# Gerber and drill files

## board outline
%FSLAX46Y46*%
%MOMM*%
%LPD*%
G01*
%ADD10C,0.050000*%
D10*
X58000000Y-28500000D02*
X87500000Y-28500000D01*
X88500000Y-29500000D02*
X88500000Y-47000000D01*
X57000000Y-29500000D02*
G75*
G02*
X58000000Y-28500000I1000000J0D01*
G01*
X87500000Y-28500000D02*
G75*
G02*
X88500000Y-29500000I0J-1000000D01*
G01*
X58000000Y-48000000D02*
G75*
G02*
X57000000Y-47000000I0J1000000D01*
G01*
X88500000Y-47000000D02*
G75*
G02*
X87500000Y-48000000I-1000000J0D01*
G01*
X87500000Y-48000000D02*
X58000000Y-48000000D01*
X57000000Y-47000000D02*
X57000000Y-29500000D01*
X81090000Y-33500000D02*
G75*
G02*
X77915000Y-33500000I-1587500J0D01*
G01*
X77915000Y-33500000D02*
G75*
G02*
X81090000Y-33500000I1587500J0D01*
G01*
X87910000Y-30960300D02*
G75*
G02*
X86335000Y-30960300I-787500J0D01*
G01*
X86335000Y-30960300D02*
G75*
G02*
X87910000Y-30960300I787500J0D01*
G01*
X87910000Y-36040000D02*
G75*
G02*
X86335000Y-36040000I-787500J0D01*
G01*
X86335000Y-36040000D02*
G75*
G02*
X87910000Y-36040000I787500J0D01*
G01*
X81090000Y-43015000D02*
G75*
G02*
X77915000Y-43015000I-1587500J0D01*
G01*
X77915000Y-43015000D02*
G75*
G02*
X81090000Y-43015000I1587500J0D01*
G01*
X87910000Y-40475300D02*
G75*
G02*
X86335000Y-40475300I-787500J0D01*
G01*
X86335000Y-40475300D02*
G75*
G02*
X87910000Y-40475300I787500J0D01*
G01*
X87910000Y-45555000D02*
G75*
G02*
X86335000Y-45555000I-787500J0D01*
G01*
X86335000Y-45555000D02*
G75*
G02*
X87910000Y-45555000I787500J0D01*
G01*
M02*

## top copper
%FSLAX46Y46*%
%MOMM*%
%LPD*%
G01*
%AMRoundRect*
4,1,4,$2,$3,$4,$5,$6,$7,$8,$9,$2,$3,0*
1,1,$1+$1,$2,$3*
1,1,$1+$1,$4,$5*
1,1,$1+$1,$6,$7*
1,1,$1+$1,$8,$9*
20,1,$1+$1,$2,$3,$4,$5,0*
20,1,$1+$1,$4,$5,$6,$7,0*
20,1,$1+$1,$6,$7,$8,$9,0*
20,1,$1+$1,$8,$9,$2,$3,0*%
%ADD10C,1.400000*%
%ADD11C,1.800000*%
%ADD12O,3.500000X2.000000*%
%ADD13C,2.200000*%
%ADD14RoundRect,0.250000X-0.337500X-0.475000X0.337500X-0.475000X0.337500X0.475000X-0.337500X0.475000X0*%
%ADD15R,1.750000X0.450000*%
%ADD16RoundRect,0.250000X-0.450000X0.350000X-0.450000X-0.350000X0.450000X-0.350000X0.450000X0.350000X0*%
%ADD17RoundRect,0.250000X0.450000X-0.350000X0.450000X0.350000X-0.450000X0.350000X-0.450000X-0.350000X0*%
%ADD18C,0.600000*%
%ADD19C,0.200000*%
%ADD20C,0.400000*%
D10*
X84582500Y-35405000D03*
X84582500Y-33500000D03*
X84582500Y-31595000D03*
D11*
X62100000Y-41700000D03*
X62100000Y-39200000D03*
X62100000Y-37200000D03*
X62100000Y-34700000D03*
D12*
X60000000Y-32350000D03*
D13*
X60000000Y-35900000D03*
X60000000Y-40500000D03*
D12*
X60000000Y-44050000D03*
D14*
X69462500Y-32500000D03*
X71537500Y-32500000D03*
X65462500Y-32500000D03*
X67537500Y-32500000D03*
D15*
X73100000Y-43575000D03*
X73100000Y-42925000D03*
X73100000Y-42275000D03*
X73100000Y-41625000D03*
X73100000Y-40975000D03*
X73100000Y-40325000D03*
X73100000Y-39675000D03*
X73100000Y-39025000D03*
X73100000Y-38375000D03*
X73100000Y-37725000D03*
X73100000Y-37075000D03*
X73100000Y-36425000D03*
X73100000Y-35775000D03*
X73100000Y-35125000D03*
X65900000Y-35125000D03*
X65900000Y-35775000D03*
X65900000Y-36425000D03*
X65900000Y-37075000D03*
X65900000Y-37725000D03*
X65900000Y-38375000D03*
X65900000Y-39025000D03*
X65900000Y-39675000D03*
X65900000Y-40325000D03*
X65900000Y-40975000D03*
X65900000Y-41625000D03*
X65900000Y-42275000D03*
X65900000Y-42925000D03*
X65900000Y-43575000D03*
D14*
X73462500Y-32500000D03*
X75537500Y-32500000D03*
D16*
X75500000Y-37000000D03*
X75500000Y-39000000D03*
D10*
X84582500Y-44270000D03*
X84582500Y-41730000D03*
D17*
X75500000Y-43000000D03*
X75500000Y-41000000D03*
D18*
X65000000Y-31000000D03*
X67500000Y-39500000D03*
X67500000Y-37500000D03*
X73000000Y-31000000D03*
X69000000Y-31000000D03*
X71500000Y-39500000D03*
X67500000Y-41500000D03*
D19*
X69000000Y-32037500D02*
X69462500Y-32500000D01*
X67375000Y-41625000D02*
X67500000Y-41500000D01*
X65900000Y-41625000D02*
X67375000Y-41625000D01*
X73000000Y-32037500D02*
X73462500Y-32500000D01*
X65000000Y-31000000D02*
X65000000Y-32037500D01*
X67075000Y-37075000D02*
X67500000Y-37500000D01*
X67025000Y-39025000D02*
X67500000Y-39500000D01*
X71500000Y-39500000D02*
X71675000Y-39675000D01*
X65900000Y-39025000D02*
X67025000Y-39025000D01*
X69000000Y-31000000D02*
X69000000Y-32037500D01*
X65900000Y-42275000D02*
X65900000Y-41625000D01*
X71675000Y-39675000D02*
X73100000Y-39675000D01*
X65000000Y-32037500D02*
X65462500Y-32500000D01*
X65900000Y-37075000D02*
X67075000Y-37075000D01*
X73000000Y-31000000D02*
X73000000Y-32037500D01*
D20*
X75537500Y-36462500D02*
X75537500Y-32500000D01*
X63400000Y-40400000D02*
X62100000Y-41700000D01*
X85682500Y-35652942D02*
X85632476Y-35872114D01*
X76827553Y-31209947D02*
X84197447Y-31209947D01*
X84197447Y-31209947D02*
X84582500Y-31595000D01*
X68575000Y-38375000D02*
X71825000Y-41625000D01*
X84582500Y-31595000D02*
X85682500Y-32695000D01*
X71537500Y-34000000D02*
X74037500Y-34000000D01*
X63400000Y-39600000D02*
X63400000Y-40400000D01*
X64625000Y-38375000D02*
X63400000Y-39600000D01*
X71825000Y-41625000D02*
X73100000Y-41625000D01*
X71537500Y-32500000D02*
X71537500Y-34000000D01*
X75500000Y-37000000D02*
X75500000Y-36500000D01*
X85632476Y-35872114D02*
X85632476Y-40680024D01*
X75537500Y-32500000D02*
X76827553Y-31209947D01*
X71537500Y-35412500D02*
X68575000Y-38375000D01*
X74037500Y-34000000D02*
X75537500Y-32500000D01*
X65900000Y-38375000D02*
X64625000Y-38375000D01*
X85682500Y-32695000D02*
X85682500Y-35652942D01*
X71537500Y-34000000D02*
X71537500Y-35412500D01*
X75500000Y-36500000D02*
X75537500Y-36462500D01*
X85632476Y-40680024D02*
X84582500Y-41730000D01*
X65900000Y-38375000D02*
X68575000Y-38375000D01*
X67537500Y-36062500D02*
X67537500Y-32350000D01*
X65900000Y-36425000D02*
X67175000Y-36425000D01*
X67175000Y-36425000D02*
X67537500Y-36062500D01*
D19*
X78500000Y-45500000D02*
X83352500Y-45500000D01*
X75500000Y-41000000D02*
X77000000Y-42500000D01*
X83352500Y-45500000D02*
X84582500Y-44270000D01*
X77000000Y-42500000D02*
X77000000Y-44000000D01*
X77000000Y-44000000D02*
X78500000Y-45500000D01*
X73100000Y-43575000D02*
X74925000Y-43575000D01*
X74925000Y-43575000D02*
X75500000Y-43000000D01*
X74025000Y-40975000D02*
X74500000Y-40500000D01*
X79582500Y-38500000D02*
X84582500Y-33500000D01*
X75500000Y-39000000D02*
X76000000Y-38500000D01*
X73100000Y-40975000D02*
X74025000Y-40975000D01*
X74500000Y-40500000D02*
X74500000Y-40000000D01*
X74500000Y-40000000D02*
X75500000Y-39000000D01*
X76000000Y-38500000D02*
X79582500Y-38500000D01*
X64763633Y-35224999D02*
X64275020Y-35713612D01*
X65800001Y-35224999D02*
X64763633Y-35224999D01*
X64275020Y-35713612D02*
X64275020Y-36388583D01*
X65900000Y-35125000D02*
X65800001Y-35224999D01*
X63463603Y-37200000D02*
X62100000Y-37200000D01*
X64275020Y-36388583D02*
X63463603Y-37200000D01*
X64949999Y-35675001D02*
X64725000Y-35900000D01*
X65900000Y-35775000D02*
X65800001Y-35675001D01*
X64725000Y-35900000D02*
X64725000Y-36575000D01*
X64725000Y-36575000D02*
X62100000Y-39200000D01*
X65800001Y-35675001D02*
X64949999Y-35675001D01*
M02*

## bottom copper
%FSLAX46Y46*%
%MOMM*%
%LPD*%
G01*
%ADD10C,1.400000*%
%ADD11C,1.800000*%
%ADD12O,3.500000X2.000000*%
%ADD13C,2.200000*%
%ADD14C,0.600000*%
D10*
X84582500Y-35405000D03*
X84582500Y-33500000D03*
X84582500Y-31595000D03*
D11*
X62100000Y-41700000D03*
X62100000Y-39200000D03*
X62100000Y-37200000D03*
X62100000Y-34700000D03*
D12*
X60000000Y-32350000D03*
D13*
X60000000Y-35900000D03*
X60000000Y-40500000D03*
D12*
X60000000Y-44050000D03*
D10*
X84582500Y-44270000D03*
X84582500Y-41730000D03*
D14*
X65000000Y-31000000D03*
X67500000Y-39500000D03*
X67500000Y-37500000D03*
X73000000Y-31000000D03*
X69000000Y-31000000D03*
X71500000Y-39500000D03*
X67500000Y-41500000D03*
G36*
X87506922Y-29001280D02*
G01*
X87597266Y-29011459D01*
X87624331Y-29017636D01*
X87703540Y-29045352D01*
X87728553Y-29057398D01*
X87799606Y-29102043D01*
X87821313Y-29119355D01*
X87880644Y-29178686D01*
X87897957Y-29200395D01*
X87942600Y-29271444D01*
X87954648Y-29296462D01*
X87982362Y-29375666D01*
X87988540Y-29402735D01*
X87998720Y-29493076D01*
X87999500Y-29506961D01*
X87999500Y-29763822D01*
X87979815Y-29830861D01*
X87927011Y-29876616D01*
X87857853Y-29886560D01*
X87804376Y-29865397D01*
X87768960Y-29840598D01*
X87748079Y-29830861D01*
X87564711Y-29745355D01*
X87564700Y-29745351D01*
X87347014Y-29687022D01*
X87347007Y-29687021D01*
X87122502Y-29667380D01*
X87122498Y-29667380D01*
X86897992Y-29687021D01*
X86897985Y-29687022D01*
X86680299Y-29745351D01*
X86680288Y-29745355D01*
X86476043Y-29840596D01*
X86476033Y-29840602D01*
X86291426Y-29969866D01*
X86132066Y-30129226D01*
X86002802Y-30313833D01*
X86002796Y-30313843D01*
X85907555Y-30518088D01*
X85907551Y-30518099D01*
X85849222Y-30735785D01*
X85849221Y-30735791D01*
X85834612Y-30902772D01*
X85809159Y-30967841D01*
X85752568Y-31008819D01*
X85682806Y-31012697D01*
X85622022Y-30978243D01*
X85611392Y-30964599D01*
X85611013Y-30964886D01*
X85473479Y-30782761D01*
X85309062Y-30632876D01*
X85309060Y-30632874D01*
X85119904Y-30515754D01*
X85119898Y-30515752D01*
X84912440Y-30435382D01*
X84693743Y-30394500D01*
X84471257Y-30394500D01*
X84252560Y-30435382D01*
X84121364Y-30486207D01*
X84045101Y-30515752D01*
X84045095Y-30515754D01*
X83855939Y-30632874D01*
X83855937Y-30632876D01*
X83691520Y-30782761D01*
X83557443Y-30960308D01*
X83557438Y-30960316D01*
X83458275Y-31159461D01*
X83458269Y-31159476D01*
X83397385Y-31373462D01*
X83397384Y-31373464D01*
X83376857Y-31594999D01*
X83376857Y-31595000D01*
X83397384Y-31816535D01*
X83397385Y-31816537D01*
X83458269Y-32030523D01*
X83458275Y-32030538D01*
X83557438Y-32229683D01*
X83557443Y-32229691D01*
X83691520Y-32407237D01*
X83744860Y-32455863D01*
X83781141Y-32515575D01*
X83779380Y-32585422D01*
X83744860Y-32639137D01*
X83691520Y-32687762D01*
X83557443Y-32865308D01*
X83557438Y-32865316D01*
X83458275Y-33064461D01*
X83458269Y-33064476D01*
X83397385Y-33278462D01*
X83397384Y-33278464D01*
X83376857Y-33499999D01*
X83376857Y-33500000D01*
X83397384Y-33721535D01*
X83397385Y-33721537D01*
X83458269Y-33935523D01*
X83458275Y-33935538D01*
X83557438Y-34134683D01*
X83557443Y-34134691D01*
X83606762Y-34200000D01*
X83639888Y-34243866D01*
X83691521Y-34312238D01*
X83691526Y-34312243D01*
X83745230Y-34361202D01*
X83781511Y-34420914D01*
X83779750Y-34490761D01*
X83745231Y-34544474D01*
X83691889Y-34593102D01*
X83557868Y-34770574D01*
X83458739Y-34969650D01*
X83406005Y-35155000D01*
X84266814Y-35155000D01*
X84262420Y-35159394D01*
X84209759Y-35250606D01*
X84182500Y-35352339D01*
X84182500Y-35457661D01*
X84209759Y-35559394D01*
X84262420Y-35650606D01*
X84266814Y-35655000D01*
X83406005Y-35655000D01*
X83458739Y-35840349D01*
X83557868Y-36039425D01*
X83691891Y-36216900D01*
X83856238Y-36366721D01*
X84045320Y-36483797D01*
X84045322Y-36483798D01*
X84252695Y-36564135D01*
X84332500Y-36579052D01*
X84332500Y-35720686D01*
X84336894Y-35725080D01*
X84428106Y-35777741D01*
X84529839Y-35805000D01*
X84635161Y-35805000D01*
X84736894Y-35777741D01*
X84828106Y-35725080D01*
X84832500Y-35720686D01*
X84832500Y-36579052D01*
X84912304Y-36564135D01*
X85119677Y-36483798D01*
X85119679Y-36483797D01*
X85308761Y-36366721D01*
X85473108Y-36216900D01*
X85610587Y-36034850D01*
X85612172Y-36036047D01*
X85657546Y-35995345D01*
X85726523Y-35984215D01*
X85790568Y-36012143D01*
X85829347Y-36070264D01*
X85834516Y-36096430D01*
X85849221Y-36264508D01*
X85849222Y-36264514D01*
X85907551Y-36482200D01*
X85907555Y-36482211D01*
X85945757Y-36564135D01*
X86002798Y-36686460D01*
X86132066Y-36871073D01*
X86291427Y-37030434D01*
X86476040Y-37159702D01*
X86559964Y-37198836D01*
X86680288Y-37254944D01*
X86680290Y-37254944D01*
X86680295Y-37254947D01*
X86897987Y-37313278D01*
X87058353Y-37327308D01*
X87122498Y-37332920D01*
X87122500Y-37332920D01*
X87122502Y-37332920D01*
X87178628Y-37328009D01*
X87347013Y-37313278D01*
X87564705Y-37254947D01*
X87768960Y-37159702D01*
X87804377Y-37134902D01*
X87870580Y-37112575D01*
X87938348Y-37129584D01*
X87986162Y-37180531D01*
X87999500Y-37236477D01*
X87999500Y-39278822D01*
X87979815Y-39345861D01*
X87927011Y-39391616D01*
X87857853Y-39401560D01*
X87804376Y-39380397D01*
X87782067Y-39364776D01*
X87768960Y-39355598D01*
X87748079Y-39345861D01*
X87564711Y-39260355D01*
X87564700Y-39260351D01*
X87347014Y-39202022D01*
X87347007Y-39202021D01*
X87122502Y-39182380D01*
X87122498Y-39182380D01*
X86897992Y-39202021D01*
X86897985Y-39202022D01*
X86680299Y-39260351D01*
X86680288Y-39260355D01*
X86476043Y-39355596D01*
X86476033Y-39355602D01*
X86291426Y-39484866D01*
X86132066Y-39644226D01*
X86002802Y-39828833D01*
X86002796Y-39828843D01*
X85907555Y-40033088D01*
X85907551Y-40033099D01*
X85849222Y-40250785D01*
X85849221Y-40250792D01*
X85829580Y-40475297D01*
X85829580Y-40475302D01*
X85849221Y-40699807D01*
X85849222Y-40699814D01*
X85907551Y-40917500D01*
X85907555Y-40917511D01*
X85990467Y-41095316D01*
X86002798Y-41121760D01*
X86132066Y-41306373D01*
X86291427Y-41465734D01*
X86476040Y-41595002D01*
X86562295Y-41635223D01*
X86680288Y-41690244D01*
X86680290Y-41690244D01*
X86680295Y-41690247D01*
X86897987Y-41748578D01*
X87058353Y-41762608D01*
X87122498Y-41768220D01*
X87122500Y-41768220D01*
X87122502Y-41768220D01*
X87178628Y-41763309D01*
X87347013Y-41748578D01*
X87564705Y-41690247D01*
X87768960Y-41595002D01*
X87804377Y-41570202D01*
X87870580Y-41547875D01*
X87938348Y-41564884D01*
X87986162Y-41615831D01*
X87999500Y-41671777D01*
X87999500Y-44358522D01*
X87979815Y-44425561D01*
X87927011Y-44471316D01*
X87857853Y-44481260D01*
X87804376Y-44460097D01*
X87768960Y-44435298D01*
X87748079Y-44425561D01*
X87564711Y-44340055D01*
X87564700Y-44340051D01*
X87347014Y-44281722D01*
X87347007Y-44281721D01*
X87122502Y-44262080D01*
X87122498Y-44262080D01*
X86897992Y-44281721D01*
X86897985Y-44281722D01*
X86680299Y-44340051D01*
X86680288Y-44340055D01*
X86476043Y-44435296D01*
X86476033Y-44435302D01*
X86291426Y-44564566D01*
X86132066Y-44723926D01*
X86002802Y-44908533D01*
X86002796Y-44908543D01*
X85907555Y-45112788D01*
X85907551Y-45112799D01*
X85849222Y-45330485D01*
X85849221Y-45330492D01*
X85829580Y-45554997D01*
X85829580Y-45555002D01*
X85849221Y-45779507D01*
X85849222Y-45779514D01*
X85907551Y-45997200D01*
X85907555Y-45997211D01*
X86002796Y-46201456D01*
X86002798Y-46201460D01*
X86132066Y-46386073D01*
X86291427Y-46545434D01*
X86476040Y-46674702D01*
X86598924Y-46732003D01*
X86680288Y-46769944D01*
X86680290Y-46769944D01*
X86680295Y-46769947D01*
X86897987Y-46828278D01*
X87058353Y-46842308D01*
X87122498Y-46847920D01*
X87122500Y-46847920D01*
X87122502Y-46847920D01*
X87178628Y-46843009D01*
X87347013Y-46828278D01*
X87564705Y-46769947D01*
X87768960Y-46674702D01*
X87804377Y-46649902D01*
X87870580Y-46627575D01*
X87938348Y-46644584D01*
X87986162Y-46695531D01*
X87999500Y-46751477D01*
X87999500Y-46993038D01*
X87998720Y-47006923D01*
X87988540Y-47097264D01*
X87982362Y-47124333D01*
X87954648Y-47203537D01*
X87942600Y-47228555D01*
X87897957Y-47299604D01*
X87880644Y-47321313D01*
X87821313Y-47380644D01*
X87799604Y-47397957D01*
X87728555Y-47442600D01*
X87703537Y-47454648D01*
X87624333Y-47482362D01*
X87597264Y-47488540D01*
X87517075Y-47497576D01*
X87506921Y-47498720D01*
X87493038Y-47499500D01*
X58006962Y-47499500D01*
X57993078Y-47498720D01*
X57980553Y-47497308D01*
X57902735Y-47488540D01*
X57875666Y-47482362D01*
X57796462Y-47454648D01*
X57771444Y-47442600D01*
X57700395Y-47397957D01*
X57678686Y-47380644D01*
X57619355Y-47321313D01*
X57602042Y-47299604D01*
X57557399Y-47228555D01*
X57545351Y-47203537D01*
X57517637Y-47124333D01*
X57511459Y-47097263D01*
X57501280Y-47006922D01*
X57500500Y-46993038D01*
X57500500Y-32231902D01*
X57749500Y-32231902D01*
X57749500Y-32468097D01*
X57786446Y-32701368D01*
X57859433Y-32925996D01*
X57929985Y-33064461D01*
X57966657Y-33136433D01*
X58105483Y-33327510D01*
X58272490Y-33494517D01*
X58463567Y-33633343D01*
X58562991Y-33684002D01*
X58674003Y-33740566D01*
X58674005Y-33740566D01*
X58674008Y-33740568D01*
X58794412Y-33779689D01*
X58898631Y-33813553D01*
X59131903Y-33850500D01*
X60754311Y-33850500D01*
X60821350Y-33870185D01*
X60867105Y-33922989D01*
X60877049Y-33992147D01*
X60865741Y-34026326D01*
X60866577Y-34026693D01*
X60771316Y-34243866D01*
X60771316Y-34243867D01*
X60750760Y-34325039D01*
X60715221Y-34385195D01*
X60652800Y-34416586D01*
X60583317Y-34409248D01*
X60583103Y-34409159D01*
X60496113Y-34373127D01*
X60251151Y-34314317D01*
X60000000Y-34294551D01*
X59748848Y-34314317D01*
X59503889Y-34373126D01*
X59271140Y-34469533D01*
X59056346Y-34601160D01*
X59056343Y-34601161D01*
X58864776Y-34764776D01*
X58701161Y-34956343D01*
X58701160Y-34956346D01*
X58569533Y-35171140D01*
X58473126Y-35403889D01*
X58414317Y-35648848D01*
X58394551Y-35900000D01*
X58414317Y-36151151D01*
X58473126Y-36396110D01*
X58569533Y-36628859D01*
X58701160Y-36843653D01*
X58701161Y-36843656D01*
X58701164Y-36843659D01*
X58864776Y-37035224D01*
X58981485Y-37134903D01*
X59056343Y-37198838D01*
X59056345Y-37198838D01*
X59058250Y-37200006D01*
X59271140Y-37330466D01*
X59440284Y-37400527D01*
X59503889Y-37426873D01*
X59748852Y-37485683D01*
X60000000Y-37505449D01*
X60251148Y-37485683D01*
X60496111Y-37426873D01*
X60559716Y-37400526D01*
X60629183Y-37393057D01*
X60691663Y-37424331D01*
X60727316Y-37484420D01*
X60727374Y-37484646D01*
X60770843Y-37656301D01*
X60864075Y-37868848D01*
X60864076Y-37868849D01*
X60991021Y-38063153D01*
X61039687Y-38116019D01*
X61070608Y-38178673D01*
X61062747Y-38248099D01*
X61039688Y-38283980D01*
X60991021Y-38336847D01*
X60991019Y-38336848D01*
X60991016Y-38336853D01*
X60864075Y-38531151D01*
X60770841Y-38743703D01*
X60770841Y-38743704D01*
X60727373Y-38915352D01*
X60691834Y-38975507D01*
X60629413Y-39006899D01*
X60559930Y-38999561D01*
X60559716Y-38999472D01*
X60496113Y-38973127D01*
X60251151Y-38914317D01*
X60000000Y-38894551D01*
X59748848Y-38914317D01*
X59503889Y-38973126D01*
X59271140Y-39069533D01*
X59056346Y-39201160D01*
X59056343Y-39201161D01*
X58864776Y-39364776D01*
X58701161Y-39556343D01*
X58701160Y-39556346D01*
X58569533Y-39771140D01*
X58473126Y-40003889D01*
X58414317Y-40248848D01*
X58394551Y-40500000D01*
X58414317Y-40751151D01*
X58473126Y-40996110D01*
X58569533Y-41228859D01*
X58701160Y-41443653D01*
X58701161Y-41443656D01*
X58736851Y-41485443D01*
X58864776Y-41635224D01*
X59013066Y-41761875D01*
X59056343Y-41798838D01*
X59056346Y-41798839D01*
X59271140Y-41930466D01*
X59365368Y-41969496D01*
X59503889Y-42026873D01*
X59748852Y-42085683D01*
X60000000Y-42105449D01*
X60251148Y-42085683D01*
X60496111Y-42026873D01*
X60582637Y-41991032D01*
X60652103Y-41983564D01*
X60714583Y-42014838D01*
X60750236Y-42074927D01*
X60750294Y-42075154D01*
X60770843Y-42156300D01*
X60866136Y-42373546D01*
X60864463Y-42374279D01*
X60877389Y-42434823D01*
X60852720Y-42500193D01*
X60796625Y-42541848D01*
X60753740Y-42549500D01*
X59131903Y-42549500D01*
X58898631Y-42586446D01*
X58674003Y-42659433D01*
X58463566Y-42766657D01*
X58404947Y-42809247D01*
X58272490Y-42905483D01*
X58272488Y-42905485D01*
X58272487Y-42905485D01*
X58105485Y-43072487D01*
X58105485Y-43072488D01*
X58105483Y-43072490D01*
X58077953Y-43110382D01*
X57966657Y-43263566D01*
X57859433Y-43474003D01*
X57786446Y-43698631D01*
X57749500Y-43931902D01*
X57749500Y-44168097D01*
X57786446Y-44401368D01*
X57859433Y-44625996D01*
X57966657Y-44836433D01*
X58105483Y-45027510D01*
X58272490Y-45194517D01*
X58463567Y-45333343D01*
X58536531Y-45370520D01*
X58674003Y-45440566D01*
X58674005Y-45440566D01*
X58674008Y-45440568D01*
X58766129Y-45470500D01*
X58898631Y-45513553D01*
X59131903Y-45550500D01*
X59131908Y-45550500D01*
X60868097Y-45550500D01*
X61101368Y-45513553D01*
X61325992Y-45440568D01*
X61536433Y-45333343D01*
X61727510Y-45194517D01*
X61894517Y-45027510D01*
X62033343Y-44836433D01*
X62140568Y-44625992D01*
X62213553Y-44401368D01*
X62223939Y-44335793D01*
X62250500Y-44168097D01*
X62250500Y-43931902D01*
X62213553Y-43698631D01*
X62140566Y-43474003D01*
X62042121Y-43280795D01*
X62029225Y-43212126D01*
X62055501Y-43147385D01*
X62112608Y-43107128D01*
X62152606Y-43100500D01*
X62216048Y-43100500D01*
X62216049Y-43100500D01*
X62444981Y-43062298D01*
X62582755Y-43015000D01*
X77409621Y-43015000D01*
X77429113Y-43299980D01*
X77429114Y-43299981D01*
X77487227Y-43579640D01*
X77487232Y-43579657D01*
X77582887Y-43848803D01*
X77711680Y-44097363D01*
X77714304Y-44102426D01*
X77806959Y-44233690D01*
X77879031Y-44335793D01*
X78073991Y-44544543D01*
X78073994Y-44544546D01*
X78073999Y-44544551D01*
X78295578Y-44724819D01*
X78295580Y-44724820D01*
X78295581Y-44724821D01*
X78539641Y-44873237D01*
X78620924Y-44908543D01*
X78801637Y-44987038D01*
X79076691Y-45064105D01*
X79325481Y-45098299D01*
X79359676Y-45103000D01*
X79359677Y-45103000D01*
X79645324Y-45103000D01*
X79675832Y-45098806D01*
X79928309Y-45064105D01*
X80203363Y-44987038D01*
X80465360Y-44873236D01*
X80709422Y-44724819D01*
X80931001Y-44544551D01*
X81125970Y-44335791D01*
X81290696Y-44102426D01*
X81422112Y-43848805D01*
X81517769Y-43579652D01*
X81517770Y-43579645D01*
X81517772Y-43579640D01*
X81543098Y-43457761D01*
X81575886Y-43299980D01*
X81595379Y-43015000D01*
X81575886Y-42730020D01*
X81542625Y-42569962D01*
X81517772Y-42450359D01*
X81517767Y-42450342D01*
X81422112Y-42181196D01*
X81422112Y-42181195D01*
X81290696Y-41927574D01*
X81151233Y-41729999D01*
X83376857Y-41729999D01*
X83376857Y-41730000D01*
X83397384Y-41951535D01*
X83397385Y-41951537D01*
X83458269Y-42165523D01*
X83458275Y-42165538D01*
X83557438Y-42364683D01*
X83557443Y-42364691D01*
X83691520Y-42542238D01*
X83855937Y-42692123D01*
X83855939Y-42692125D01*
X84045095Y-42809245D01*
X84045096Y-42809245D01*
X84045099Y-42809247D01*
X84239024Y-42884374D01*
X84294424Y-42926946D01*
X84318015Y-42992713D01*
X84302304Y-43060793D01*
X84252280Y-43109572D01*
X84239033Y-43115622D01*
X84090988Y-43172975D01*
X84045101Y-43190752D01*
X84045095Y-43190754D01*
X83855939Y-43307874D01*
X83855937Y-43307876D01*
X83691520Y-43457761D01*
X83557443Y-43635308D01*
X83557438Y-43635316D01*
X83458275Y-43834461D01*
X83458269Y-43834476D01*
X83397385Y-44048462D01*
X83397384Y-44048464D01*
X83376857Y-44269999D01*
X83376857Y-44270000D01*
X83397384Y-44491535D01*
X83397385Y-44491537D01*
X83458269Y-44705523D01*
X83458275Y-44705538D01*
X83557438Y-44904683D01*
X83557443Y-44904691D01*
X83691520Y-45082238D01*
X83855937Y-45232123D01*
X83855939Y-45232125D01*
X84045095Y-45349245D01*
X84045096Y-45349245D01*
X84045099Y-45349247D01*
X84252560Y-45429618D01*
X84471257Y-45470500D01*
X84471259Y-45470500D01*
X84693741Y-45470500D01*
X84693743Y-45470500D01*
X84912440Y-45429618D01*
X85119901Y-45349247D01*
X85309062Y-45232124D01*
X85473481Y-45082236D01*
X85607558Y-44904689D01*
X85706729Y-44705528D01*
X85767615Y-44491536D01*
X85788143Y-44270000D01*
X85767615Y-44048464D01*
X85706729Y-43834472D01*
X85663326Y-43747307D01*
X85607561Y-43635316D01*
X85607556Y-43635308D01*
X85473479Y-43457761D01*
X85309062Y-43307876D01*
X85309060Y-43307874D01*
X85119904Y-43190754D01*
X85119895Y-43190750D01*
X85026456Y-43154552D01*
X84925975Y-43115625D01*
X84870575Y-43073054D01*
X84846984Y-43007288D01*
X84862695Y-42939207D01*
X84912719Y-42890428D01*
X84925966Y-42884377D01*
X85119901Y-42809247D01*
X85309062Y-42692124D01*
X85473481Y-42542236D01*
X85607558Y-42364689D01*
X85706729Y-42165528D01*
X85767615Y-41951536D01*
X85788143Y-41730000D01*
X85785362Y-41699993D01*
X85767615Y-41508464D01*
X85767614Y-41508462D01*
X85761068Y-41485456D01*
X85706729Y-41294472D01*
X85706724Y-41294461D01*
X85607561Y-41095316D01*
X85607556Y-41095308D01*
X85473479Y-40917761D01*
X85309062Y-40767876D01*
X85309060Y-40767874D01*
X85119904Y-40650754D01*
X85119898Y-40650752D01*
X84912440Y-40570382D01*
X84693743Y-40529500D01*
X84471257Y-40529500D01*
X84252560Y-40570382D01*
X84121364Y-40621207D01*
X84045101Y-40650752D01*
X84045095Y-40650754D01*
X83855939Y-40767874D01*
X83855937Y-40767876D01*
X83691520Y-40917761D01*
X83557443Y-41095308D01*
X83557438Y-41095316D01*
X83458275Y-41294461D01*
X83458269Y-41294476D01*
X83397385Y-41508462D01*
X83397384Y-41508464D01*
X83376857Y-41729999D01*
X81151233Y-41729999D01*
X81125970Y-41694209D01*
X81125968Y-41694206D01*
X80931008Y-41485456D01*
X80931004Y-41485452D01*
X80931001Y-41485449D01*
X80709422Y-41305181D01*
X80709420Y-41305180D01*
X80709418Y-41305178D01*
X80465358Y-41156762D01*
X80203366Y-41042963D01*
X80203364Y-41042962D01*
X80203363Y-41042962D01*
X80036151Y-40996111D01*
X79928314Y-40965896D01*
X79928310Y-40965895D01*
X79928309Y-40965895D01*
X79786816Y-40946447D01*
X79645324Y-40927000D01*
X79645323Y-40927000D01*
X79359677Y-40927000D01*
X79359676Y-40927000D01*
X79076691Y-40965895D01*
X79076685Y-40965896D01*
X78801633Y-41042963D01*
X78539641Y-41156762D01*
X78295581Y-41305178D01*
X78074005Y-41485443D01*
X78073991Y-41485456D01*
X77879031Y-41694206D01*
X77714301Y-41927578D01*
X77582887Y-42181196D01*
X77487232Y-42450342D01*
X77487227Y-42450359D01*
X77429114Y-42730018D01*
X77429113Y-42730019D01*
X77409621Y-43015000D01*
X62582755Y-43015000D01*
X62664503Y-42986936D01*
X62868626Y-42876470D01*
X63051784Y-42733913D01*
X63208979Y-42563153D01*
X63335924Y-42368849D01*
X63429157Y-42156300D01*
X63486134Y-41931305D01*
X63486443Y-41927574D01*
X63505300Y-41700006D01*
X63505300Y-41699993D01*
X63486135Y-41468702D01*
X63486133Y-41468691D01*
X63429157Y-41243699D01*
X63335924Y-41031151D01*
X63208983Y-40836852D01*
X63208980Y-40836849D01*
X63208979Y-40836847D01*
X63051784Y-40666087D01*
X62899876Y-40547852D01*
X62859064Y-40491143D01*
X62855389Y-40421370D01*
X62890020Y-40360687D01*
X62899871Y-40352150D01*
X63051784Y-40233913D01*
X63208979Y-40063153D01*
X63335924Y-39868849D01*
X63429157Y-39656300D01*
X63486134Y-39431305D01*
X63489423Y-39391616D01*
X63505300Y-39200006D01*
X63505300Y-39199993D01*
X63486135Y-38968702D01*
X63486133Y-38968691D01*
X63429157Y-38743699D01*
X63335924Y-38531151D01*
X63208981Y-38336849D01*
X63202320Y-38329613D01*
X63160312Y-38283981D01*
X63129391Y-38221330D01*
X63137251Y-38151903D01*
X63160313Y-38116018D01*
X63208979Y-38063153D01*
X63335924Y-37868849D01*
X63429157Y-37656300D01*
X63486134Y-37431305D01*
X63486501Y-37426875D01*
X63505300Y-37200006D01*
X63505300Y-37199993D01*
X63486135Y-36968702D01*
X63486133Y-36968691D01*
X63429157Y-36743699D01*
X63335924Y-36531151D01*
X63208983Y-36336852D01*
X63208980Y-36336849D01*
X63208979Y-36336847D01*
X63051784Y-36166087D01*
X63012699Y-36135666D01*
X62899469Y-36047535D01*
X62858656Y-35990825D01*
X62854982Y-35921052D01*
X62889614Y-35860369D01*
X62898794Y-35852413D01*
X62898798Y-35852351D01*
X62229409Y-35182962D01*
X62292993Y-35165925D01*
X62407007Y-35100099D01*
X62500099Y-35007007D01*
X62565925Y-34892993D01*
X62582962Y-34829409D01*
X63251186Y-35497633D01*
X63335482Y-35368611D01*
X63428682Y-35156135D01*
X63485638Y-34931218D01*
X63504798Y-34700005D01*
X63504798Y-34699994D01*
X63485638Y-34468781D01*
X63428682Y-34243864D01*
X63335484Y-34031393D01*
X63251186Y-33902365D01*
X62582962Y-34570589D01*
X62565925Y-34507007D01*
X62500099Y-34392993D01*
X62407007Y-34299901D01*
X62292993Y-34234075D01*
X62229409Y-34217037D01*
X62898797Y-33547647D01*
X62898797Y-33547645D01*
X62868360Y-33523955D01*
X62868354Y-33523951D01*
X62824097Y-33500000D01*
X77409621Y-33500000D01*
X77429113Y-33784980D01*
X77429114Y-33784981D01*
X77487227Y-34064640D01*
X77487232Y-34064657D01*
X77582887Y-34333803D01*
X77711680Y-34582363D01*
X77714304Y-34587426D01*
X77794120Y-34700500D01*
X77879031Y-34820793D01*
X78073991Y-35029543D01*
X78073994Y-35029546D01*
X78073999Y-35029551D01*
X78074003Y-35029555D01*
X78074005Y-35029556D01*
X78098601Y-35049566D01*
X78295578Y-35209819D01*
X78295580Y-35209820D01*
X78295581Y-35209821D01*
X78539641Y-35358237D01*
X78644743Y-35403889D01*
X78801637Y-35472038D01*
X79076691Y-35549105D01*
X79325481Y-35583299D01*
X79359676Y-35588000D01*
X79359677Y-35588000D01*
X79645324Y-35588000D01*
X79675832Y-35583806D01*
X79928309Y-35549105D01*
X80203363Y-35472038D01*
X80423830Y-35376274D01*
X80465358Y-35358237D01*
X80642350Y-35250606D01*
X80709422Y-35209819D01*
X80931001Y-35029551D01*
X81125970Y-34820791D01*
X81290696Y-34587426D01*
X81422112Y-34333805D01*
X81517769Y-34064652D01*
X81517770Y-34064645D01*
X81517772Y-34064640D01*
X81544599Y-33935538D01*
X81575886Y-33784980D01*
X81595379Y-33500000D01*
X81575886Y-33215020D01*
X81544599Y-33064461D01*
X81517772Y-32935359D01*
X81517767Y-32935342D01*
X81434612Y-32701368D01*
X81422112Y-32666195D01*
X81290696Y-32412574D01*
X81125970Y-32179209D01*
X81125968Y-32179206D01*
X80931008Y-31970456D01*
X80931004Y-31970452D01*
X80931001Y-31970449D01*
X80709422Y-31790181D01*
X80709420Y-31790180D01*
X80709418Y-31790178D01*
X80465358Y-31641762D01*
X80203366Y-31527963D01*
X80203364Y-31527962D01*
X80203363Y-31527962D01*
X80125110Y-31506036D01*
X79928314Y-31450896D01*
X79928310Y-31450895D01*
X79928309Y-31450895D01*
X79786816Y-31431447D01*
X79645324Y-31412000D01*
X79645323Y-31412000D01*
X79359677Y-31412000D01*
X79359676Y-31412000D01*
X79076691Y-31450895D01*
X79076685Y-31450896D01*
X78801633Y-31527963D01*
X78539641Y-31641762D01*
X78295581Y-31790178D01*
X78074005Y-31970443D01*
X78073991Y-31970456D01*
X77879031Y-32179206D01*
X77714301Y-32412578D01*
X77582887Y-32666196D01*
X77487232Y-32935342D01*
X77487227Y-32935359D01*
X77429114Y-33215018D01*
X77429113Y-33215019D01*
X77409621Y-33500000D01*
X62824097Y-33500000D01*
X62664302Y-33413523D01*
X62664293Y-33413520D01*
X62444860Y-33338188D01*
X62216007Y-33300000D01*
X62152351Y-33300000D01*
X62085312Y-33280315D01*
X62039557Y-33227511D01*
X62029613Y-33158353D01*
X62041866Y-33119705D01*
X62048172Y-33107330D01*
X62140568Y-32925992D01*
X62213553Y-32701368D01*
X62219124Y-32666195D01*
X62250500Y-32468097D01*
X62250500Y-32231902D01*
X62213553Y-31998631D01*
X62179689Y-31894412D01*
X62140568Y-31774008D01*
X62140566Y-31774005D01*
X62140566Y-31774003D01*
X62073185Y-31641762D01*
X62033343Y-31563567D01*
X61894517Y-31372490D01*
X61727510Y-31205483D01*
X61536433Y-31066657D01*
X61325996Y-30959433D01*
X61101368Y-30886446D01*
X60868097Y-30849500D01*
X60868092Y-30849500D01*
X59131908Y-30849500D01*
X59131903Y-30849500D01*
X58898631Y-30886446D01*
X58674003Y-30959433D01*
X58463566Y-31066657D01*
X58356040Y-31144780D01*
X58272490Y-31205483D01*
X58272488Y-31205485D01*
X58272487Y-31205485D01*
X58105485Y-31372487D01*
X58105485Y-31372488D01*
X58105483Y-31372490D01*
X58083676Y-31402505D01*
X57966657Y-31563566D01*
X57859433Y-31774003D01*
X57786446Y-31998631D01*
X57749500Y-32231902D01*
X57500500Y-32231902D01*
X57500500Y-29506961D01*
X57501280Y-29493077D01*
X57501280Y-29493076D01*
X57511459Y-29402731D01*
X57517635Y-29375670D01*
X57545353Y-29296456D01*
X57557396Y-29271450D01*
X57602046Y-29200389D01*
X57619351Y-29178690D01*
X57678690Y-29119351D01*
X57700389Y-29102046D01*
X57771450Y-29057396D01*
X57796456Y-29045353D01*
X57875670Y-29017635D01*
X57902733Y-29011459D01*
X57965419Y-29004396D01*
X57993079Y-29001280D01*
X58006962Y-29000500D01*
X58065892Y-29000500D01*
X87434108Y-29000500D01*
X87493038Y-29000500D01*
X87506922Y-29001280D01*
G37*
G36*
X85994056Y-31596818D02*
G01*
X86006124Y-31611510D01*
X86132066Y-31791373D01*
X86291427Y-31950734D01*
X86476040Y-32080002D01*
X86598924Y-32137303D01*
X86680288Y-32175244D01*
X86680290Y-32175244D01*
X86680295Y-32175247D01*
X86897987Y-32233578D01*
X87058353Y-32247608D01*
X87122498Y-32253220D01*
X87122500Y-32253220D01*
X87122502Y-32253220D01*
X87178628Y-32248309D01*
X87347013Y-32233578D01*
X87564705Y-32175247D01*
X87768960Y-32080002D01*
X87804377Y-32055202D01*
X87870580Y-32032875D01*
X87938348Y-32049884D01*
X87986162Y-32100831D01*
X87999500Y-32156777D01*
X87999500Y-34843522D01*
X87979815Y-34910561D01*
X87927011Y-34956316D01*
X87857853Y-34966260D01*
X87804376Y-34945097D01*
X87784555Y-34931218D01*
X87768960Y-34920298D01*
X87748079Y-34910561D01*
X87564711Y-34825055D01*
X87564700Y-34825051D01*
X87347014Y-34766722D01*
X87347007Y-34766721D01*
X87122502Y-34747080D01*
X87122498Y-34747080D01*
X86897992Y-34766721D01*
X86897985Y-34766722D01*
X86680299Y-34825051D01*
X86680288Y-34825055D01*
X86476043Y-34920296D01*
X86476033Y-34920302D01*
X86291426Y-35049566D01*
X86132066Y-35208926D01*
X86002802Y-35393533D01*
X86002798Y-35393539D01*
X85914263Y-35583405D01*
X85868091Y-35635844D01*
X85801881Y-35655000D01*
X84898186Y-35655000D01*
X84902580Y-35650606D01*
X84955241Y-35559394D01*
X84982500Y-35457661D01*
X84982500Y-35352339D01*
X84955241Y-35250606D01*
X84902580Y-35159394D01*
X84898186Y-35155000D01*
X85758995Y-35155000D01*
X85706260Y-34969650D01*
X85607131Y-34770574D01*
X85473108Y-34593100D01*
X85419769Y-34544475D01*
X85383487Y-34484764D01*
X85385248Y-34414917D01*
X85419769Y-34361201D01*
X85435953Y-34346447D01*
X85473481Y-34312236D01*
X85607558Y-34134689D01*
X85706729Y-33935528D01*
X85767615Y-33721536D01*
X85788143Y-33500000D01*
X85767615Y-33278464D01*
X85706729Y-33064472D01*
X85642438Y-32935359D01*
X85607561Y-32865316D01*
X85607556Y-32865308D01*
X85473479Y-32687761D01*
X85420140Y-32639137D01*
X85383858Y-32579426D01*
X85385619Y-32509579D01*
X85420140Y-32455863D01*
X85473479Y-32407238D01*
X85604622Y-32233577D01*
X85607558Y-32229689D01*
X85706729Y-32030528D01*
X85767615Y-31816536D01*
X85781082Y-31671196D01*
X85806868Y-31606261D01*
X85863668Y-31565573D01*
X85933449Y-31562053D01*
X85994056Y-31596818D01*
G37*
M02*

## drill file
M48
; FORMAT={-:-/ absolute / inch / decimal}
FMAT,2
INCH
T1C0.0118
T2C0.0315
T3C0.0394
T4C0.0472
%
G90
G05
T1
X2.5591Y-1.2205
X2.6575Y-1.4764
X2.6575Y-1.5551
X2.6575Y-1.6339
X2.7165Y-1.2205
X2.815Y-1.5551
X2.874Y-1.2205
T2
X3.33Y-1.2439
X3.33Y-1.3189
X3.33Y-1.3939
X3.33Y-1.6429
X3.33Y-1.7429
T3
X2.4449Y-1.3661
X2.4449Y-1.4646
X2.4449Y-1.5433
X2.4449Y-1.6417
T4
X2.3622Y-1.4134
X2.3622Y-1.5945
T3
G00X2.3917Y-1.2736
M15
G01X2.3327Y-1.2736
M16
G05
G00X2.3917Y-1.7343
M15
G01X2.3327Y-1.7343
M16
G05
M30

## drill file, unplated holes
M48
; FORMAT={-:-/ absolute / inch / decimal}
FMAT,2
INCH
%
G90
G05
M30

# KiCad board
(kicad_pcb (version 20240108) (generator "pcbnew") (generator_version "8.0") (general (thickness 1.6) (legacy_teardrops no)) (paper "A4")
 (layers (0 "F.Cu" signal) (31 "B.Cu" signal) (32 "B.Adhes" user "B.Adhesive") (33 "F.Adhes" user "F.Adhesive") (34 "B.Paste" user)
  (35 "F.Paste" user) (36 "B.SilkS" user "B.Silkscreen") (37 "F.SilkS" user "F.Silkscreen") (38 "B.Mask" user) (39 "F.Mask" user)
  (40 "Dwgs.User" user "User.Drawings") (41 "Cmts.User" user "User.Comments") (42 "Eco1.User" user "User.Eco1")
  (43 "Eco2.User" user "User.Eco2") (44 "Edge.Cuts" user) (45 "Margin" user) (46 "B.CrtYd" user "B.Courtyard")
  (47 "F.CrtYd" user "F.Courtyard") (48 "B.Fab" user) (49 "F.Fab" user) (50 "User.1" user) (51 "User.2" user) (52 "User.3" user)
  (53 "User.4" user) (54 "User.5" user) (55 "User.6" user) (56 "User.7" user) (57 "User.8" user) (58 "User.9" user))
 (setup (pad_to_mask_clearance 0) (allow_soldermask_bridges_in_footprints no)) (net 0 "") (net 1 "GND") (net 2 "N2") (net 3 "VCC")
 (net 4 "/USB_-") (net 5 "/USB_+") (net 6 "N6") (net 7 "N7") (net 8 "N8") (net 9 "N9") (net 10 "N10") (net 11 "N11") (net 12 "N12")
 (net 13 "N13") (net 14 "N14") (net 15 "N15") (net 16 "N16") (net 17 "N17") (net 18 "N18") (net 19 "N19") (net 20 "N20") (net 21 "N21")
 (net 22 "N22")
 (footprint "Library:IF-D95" (layer "F.Cu") (at 88.0675 30.0075 -90)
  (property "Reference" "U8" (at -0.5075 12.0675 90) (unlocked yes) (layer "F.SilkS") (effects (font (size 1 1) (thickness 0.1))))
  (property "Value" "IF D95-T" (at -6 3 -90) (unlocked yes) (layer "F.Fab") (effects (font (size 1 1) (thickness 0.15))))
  (fp_circle (center 3.4925 8.565) (end 5.08 8.565) (stroke (width 0.05) (type default)) (fill none) (layer "Edge.Cuts"))
  (fp_circle (center 0.9528 0.945) (end 1.7403 0.945) (stroke (width 0.05) (type default)) (fill none) (layer "Edge.Cuts"))
  (fp_circle (center 6.0325 0.945) (end 6.82 0.945) (stroke (width 0.05) (type default)) (fill none) (layer "Edge.Cuts"))
  (pad "1" thru_hole circle (at 5.3975 3.485 270) (size 1.4 1.4) (drill 0.8) (layers "*.Cu" "*.Mask") (remove_unused_layers no)
   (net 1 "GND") (thermal_bridge_angle 90))
  (pad "2" thru_hole circle (at 3.4925 3.485 270) (size 1.4 1.4) (drill 0.8) (layers "*.Cu" "*.Mask") (remove_unused_layers no) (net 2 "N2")
   (thermal_bridge_angle 90))
  (pad "3" thru_hole circle (at 1.5875 3.485 270) (size 1.4 1.4) (drill 0.8) (layers "*.Cu" "*.Mask") (remove_unused_layers no)
   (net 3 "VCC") (thermal_bridge_angle 90)))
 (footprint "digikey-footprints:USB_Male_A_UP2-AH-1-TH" (layer "F.Cu") (at 60 38.2 -90)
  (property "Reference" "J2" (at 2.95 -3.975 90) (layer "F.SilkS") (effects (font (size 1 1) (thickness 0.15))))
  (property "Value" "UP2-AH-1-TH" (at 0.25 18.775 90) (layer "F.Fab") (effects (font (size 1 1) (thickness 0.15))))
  (pad "1" thru_hole circle (at 3.5 -2.1 270) (size 1.8 1.8) (drill 1) (layers "*.Cu" "*.Mask") (remove_unused_layers no) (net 3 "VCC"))
  (pad "2" thru_hole circle (at 1 -2.1 270) (size 1.8 1.8) (drill 1) (layers "*.Cu" "*.Mask") (remove_unused_layers no) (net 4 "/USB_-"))
  (pad "3" thru_hole circle (at -1 -2.1 270) (size 1.8 1.8) (drill 1) (layers "*.Cu" "*.Mask") (remove_unused_layers no) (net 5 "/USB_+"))
  (pad "4" thru_hole circle (at -3.5 -2.1 270) (size 1.8 1.8) (drill 1) (layers "*.Cu" "*.Mask") (remove_unused_layers no) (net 1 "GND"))
  (pad "SH" thru_hole oval (at -5.85 0 270) (size 2 3.5) (drill oval 1 2.5) (layers "*.Cu" "*.Mask") (remove_unused_layers no))
  (pad "SH" thru_hole circle (at -2.3 0 270) (size 2.2 2.2) (drill 1.2) (layers "*.Cu" "*.Mask") (remove_unused_layers no))
  (pad "SH" thru_hole circle (at 2.3 0 270) (size 2.2 2.2) (drill 1.2) (layers "*.Cu" "*.Mask") (remove_unused_layers no))
  (pad "SH" thru_hole oval (at 5.85 0 270) (size 2 3.5) (drill oval 1 2.5) (layers "*.Cu" "*.Mask") (remove_unused_layers no)))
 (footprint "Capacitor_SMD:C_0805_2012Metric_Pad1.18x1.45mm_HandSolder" (layer "F.Cu") (at 70.5 32.5)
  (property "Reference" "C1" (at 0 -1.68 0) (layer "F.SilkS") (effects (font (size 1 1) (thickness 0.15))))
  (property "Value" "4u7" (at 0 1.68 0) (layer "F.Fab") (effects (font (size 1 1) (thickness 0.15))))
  (pad "1" smd roundrect (at -1.0375 0) (size 1.175 1.45) (layers "F.Cu" "F.Paste" "F.Mask") (roundrect_rratio 0.212766) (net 1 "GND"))
  (pad "2" smd roundrect (at 1.0375 0) (size 1.175 1.45) (layers "F.Cu" "F.Paste" "F.Mask") (roundrect_rratio 0.212766) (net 3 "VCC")))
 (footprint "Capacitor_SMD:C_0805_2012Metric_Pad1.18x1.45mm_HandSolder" (layer "F.Cu") (at 66.5 32.5)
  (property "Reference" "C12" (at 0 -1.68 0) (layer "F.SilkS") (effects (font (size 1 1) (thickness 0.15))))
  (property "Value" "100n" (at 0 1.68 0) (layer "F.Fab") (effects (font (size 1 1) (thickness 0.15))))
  (pad "1" smd roundrect (at -1.0375 0) (size 1.175 1.45) (layers "F.Cu" "F.Paste" "F.Mask") (roundrect_rratio 0.212766) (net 1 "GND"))
  (pad "2" smd roundrect (at 1.0375 0) (size 1.175 1.45) (layers "F.Cu" "F.Paste" "F.Mask") (roundrect_rratio 0.212766) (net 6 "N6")))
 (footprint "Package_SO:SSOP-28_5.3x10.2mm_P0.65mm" (layer "F.Cu") (at 69.5 39.35 180)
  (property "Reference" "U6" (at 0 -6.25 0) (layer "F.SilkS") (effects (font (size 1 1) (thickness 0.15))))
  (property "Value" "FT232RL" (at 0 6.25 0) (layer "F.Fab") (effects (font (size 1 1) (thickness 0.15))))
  (pad "1" smd rect (at -3.6 -4.225 180) (size 1.75 0.45) (layers "F.Cu" "F.Paste" "F.Mask") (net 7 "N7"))
  (pad "2" smd rect (at -3.6 -3.575 180) (size 1.75 0.45) (layers "F.Cu" "F.Paste" "F.Mask") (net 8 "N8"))
  (pad "3" smd rect (at -3.6 -2.925 180) (size 1.75 0.45) (layers "F.Cu" "F.Paste" "F.Mask") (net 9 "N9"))
  (pad "4" smd rect (at -3.6 -2.275 180) (size 1.75 0.45) (layers "F.Cu" "F.Paste" "F.Mask") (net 3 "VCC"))
  (pad "5" smd rect (at -3.6 -1.625 180) (size 1.75 0.45) (layers "F.Cu" "F.Paste" "F.Mask") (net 2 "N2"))
  (pad "6" smd rect (at -3.6 -0.975 180) (size 1.75 0.45) (layers "F.Cu" "F.Paste" "F.Mask") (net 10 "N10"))
  (pad "7" smd rect (at -3.6 -0.325 180) (size 1.75 0.45) (layers "F.Cu" "F.Paste" "F.Mask") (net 1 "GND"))
  (pad "8" smd rect (at -3.6 0.325 180) (size 1.75 0.45) (layers "F.Cu" "F.Paste" "F.Mask"))
  (pad "9" smd rect (at -3.6 0.975 180) (size 1.75 0.45) (layers "F.Cu" "F.Paste" "F.Mask") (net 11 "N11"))
  (pad "10" smd rect (at -3.6 1.625 180) (size 1.75 0.45) (layers "F.Cu" "F.Paste" "F.Mask") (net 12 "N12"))
  (pad "11" smd rect (at -3.6 2.275 180) (size 1.75 0.45) (layers "F.Cu" "F.Paste" "F.Mask") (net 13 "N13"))
  (pad "12" smd rect (at -3.6 2.925 180) (size 1.75 0.45) (layers "F.Cu" "F.Paste" "F.Mask") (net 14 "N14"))
  (pad "13" smd rect (at -3.6 3.575 180) (size 1.75 0.45) (layers "F.Cu" "F.Paste" "F.Mask") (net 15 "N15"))
  (pad "14" smd rect (at -3.6 4.225 180) (size 1.75 0.45) (layers "F.Cu" "F.Paste" "F.Mask") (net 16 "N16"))
  (pad "15" smd rect (at 3.6 4.225 180) (size 1.75 0.45) (layers "F.Cu" "F.Paste" "F.Mask") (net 5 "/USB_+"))
  (pad "16" smd rect (at 3.6 3.575 180) (size 1.75 0.45) (layers "F.Cu" "F.Paste" "F.Mask") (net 4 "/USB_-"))
  (pad "17" smd rect (at 3.6 2.925 180) (size 1.75 0.45) (layers "F.Cu" "F.Paste" "F.Mask") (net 6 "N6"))
  (pad "18" smd rect (at 3.6 2.275 180) (size 1.75 0.45) (layers "F.Cu" "F.Paste" "F.Mask") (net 1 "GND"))
  (pad "19" smd rect (at 3.6 1.625 180) (size 1.75 0.45) (layers "F.Cu" "F.Paste" "F.Mask") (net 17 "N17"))
  (pad "20" smd rect (at 3.6 0.975 180) (size 1.75 0.45) (layers "F.Cu" "F.Paste" "F.Mask") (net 3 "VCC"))
  (pad "21" smd rect (at 3.6 0.325 180) (size 1.75 0.45) (layers "F.Cu" "F.Paste" "F.Mask") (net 1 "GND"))
  (pad "22" smd rect (at 3.6 -0.325 180) (size 1.75 0.45) (layers "F.Cu" "F.Paste" "F.Mask") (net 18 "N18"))
  (pad "23" smd rect (at 3.6 -0.975 180) (size 1.75 0.45) (layers "F.Cu" "F.Paste" "F.Mask") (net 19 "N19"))
  (pad "24" smd rect (at 3.6 -1.625 180) (size 1.75 0.45) (layers "F.Cu" "F.Paste" "F.Mask"))
  (pad "25" smd rect (at 3.6 -2.275 180) (size 1.75 0.45) (layers "F.Cu" "F.Paste" "F.Mask") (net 1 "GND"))
  (pad "26" smd rect (at 3.6 -2.925 180) (size 1.75 0.45) (layers "F.Cu" "F.Paste" "F.Mask") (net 1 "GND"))
  (pad "27" smd rect (at 3.6 -3.575 180) (size 1.75 0.45) (layers "F.Cu" "F.Paste" "F.Mask") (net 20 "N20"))
  (pad "28" smd rect (at 3.6 -4.225 180) (size 1.75 0.45) (layers "F.Cu" "F.Paste" "F.Mask") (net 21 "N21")))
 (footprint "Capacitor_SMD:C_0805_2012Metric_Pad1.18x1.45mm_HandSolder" (layer "F.Cu") (at 74.5 32.5)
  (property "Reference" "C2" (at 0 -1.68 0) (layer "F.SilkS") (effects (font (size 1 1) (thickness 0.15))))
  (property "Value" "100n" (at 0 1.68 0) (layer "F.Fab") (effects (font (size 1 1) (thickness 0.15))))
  (pad "1" smd roundrect (at -1.0375 0) (size 1.175 1.45) (layers "F.Cu" "F.Paste" "F.Mask") (roundrect_rratio 0.212766) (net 1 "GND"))
  (pad "2" smd roundrect (at 1.0375 0) (size 1.175 1.45) (layers "F.Cu" "F.Paste" "F.Mask") (roundrect_rratio 0.212766) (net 3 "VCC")))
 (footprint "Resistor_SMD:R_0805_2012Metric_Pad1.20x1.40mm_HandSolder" (layer "F.Cu") (at 75.5 38 -90)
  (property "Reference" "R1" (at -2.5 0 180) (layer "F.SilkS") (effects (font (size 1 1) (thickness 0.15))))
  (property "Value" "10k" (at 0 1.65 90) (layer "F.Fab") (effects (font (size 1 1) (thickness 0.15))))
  (pad "1" smd roundrect (at -1 0 270) (size 1.2 1.4) (layers "F.Cu" "F.Paste" "F.Mask") (roundrect_rratio 0.208333) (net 3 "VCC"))
  (pad "2" smd roundrect (at 1 0 270) (size 1.2 1.4) (layers "F.Cu" "F.Paste" "F.Mask") (roundrect_rratio 0.208333) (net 2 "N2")))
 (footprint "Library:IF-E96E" (layer "F.Cu") (at 88.0675 39.5075 -90)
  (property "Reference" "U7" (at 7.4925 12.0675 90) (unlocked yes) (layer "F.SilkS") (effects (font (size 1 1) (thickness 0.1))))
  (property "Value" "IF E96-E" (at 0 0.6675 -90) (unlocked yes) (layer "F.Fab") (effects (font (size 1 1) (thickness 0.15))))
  (fp_circle (center 3.5075 8.565) (end 5.095 8.565) (stroke (width 0.05) (type default)) (fill none) (layer "Edge.Cuts"))
  (fp_circle (center 0.9678 0.945) (end 1.7553 0.945) (stroke (width 0.05) (type default)) (fill none) (layer "Edge.Cuts"))
  (fp_circle (center 6.0475 0.945) (end 6.835 0.945) (stroke (width 0.05) (type default)) (fill none) (layer "Edge.Cuts"))
  (pad "1" thru_hole circle (at 4.7625 3.485 270) (size 1.4 1.4) (drill 0.8) (layers "*.Cu" "*.Mask") (remove_unused_layers no)
   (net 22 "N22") (thermal_bridge_angle 90))
  (pad "2" thru_hole circle (at 2.2225 3.485 270) (size 1.4 1.4) (drill 0.8) (layers "*.Cu" "*.Mask") (remove_unused_layers no)
   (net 3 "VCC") (thermal_bridge_angle 90)))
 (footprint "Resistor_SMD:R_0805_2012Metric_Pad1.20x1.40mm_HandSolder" (layer "F.Cu") (at 75.5 42 90)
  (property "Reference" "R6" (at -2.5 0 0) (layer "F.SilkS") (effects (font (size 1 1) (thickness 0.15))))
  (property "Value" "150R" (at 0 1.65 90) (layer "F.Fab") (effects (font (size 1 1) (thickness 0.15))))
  (pad "1" smd roundrect (at -1 0 90) (size 1.2 1.4) (layers "F.Cu" "F.Paste" "F.Mask") (roundrect_rratio 0.208333) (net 7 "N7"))
  (pad "2" smd roundrect (at 1 0 90) (size 1.2 1.4) (layers "F.Cu" "F.Paste" "F.Mask") (roundrect_rratio 0.208333) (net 22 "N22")))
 (gr_line (start 58 28.5) (end 87.5 28.5) (stroke (width 0.05) (type default)) (layer "Edge.Cuts"))
 (gr_line (start 88.5 29.5) (end 88.5 47) (stroke (width 0.05) (type default)) (layer "Edge.Cuts"))
 (gr_arc (start 57 29.5) (mid 57.292893 28.792893) (end 58 28.5) (stroke (width 0.05) (type default)) (layer "Edge.Cuts"))
 (gr_arc (start 87.5 28.5) (mid 88.207107 28.792893) (end 88.5 29.5) (stroke (width 0.05) (type default)) (layer "Edge.Cuts"))
 (gr_arc (start 58 48) (mid 57.292893 47.707107) (end 57 47) (stroke (width 0.05) (type default)) (layer "Edge.Cuts"))
 (gr_arc (start 88.5 47) (mid 88.207107 47.707107) (end 87.5 48) (stroke (width 0.05) (type default)) (layer "Edge.Cuts"))
 (gr_line (start 87.5 48) (end 58 48) (stroke (width 0.05) (type default)) (layer "Edge.Cuts"))
 (gr_line (start 57 47) (end 57 29.5) (stroke (width 0.05) (type default)) (layer "Edge.Cuts"))
 (segment (start 69 32.0375) (end 69.4625 32.5) (width 0.2) (layer "F.Cu") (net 1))
 (segment (start 67.375 41.625) (end 67.5 41.5) (width 0.2) (layer "F.Cu") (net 1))
 (segment (start 65.9 41.625) (end 67.375 41.625) (width 0.2) (layer "F.Cu") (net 1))
 (segment (start 73 32.0375) (end 73.4625 32.5) (width 0.2) (layer "F.Cu") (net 1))
 (segment (start 65 31) (end 65 32.0375) (width 0.2) (layer "F.Cu") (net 1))
 (segment (start 67.075 37.075) (end 67.5 37.5) (width 0.2) (layer "F.Cu") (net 1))
 (segment (start 67.025 39.025) (end 67.5 39.5) (width 0.2) (layer "F.Cu") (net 1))
 (segment (start 71.5 39.5) (end 71.675 39.675) (width 0.2) (layer "F.Cu") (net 1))
 (segment (start 65.9 39.025) (end 67.025 39.025) (width 0.2) (layer "F.Cu") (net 1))
 (segment (start 69 31) (end 69 32.0375) (width 0.2) (layer "F.Cu") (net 1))
 (segment (start 65.9 42.275) (end 65.9 41.625) (width 0.2) (layer "F.Cu") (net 1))
 (segment (start 71.675 39.675) (end 73.1 39.675) (width 0.2) (layer "F.Cu") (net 1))
 (segment (start 65 32.0375) (end 65.4625 32.5) (width 0.2) (layer "F.Cu") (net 1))
 (segment (start 65.9 37.075) (end 67.075 37.075) (width 0.2) (layer "F.Cu") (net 1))
 (segment (start 73 31) (end 73 32.0375) (width 0.2) (layer "F.Cu") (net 1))
 (via (at 65 31) (size 0.6) (drill 0.3) (layers "F.Cu" "B.Cu") (free yes) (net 1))
 (via (at 67.5 39.5) (size 0.6) (drill 0.3) (layers "F.Cu" "B.Cu") (free yes) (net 1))
 (via (at 67.5 37.5) (size 0.6) (drill 0.3) (layers "F.Cu" "B.Cu") (free yes) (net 1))
 (via (at 73 31) (size 0.6) (drill 0.3) (layers "F.Cu" "B.Cu") (free yes) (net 1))
 (via (at 69 31) (size 0.6) (drill 0.3) (layers "F.Cu" "B.Cu") (free yes) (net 1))
 (via (at 71.5 39.5) (size 0.6) (drill 0.3) (layers "F.Cu" "B.Cu") (free yes) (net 1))
 (via (at 67.5 41.5) (size 0.6) (drill 0.3) (layers "F.Cu" "B.Cu") (free yes) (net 1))
 (segment (start 75.5375 36.4625) (end 75.5375 32.5) (width 0.4) (layer "F.Cu") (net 3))
 (segment (start 63.4 40.4) (end 62.1 41.7) (width 0.4) (layer "F.Cu") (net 3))
 (segment (start 85.6825 35.652942) (end 85.632476 35.872114) (width 0.4) (layer "F.Cu") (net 3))
 (segment (start 76.827553 31.209947) (end 84.197447 31.209947) (width 0.4) (layer "F.Cu") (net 3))
 (segment (start 84.197447 31.209947) (end 84.5825 31.595) (width 0.4) (layer "F.Cu") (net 3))
 (segment (start 68.575 38.375) (end 71.825 41.625) (width 0.4) (layer "F.Cu") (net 3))
 (segment (start 84.5825 31.595) (end 85.6825 32.695) (width 0.4) (layer "F.Cu") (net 3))
 (segment (start 71.5375 34) (end 74.0375 34) (width 0.4) (layer "F.Cu") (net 3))
 (segment (start 63.4 39.6) (end 63.4 40.4) (width 0.4) (layer "F.Cu") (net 3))
 (segment (start 64.625 38.375) (end 63.4 39.6) (width 0.4) (layer "F.Cu") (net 3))
 (segment (start 71.825 41.625) (end 73.1 41.625) (width 0.4) (layer "F.Cu") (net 3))
 (segment (start 71.5375 32.5) (end 71.5375 34) (width 0.4) (layer "F.Cu") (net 3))
 (segment (start 75.5 37) (end 75.5 36.5) (width 0.4) (layer "F.Cu") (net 3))
 (segment (start 85.632476 35.872114) (end 85.632476 40.680024) (width 0.4) (layer "F.Cu") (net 3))
 (segment (start 75.5375 32.5) (end 76.827553 31.209947) (width 0.4) (layer "F.Cu") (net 3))
 (segment (start 71.5375 35.4125) (end 68.575 38.375) (width 0.4) (layer "F.Cu") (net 3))
 (segment (start 74.0375 34) (end 75.5375 32.5) (width 0.4) (layer "F.Cu") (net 3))
 (segment (start 65.9 38.375) (end 64.625 38.375) (width 0.4) (layer "F.Cu") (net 3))
 (segment (start 85.6825 32.695) (end 85.6825 35.652942) (width 0.4) (layer "F.Cu") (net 3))
 (segment (start 71.5375 34) (end 71.5375 35.4125) (width 0.4) (layer "F.Cu") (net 3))
 (segment (start 75.5 36.5) (end 75.5375 36.4625) (width 0.4) (layer "F.Cu") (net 3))
 (segment (start 85.632476 40.680024) (end 84.5825 41.73) (width 0.4) (layer "F.Cu") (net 3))
 (segment (start 65.9 38.375) (end 68.575 38.375) (width 0.4) (layer "F.Cu") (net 3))
 (segment (start 67.5375 36.0625) (end 67.5375 32.35) (width 0.4) (layer "F.Cu") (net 6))
 (segment (start 65.9 36.425) (end 67.175 36.425) (width 0.4) (layer "F.Cu") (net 6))
 (segment (start 67.175 36.425) (end 67.5375 36.0625) (width 0.4) (layer "F.Cu") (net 6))
 (segment (start 78.5 45.5) (end 83.3525 45.5) (width 0.2) (layer "F.Cu") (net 22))
 (segment (start 75.5 41) (end 77 42.5) (width 0.2) (layer "F.Cu") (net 22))
 (segment (start 83.3525 45.5) (end 84.5825 44.27) (width 0.2) (layer "F.Cu") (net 22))
 (segment (start 77 42.5) (end 77 44) (width 0.2) (layer "F.Cu") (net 22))
 (segment (start 77 44) (end 78.5 45.5) (width 0.2) (layer "F.Cu") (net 22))
 (segment (start 73.1 43.575) (end 74.925 43.575) (width 0.2) (layer "F.Cu") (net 7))
 (segment (start 74.925 43.575) (end 75.5 43) (width 0.2) (layer "F.Cu") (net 7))
 (segment (start 74.025 40.975) (end 74.5 40.5) (width 0.2) (layer "F.Cu") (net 2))
 (segment (start 79.5825 38.5) (end 84.5825 33.5) (width 0.2) (layer "F.Cu") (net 2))
 (segment (start 75.5 39) (end 76 38.5) (width 0.2) (layer "F.Cu") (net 2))
 (segment (start 73.1 40.975) (end 74.025 40.975) (width 0.2) (layer "F.Cu") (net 2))
 (segment (start 74.5 40.5) (end 74.5 40) (width 0.2) (layer "F.Cu") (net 2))
 (segment (start 74.5 40) (end 75.5 39) (width 0.2) (layer "F.Cu") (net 2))
 (segment (start 76 38.5) (end 79.5825 38.5) (width 0.2) (layer "F.Cu") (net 2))
 (segment (start 64.763633 35.224999) (end 64.27502 35.713612) (width 0.2) (layer "F.Cu") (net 5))
 (segment (start 65.800001 35.224999) (end 64.763633 35.224999) (width 0.2) (layer "F.Cu") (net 5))
 (segment (start 64.27502 35.713612) (end 64.27502 36.388583) (width 0.2) (layer "F.Cu") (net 5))
 (segment (start 65.9 35.125) (end 65.800001 35.224999) (width 0.2) (layer "F.Cu") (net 5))
 (segment (start 63.463603 37.2) (end 62.1 37.2) (width 0.2) (layer "F.Cu") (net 5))
 (segment (start 64.27502 36.388583) (end 63.463603 37.2) (width 0.2) (layer "F.Cu") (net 5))
 (segment (start 64.949999 35.675001) (end 64.725 35.9) (width 0.2) (layer "F.Cu") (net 4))
 (segment (start 65.9 35.775) (end 65.800001 35.675001) (width 0.2) (layer "F.Cu") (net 4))
 (segment (start 64.725 35.9) (end 64.725 36.575) (width 0.2) (layer "F.Cu") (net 4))
 (segment (start 64.725 36.575) (end 62.1 39.2) (width 0.2) (layer "F.Cu") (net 4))
 (segment (start 65.800001 35.675001) (end 64.949999 35.675001) (width 0.2) (layer "F.Cu") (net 4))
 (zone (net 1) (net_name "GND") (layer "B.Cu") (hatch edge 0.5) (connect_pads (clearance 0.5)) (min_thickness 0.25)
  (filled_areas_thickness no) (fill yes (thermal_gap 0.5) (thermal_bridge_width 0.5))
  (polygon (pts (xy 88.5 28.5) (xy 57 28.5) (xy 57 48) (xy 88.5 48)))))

